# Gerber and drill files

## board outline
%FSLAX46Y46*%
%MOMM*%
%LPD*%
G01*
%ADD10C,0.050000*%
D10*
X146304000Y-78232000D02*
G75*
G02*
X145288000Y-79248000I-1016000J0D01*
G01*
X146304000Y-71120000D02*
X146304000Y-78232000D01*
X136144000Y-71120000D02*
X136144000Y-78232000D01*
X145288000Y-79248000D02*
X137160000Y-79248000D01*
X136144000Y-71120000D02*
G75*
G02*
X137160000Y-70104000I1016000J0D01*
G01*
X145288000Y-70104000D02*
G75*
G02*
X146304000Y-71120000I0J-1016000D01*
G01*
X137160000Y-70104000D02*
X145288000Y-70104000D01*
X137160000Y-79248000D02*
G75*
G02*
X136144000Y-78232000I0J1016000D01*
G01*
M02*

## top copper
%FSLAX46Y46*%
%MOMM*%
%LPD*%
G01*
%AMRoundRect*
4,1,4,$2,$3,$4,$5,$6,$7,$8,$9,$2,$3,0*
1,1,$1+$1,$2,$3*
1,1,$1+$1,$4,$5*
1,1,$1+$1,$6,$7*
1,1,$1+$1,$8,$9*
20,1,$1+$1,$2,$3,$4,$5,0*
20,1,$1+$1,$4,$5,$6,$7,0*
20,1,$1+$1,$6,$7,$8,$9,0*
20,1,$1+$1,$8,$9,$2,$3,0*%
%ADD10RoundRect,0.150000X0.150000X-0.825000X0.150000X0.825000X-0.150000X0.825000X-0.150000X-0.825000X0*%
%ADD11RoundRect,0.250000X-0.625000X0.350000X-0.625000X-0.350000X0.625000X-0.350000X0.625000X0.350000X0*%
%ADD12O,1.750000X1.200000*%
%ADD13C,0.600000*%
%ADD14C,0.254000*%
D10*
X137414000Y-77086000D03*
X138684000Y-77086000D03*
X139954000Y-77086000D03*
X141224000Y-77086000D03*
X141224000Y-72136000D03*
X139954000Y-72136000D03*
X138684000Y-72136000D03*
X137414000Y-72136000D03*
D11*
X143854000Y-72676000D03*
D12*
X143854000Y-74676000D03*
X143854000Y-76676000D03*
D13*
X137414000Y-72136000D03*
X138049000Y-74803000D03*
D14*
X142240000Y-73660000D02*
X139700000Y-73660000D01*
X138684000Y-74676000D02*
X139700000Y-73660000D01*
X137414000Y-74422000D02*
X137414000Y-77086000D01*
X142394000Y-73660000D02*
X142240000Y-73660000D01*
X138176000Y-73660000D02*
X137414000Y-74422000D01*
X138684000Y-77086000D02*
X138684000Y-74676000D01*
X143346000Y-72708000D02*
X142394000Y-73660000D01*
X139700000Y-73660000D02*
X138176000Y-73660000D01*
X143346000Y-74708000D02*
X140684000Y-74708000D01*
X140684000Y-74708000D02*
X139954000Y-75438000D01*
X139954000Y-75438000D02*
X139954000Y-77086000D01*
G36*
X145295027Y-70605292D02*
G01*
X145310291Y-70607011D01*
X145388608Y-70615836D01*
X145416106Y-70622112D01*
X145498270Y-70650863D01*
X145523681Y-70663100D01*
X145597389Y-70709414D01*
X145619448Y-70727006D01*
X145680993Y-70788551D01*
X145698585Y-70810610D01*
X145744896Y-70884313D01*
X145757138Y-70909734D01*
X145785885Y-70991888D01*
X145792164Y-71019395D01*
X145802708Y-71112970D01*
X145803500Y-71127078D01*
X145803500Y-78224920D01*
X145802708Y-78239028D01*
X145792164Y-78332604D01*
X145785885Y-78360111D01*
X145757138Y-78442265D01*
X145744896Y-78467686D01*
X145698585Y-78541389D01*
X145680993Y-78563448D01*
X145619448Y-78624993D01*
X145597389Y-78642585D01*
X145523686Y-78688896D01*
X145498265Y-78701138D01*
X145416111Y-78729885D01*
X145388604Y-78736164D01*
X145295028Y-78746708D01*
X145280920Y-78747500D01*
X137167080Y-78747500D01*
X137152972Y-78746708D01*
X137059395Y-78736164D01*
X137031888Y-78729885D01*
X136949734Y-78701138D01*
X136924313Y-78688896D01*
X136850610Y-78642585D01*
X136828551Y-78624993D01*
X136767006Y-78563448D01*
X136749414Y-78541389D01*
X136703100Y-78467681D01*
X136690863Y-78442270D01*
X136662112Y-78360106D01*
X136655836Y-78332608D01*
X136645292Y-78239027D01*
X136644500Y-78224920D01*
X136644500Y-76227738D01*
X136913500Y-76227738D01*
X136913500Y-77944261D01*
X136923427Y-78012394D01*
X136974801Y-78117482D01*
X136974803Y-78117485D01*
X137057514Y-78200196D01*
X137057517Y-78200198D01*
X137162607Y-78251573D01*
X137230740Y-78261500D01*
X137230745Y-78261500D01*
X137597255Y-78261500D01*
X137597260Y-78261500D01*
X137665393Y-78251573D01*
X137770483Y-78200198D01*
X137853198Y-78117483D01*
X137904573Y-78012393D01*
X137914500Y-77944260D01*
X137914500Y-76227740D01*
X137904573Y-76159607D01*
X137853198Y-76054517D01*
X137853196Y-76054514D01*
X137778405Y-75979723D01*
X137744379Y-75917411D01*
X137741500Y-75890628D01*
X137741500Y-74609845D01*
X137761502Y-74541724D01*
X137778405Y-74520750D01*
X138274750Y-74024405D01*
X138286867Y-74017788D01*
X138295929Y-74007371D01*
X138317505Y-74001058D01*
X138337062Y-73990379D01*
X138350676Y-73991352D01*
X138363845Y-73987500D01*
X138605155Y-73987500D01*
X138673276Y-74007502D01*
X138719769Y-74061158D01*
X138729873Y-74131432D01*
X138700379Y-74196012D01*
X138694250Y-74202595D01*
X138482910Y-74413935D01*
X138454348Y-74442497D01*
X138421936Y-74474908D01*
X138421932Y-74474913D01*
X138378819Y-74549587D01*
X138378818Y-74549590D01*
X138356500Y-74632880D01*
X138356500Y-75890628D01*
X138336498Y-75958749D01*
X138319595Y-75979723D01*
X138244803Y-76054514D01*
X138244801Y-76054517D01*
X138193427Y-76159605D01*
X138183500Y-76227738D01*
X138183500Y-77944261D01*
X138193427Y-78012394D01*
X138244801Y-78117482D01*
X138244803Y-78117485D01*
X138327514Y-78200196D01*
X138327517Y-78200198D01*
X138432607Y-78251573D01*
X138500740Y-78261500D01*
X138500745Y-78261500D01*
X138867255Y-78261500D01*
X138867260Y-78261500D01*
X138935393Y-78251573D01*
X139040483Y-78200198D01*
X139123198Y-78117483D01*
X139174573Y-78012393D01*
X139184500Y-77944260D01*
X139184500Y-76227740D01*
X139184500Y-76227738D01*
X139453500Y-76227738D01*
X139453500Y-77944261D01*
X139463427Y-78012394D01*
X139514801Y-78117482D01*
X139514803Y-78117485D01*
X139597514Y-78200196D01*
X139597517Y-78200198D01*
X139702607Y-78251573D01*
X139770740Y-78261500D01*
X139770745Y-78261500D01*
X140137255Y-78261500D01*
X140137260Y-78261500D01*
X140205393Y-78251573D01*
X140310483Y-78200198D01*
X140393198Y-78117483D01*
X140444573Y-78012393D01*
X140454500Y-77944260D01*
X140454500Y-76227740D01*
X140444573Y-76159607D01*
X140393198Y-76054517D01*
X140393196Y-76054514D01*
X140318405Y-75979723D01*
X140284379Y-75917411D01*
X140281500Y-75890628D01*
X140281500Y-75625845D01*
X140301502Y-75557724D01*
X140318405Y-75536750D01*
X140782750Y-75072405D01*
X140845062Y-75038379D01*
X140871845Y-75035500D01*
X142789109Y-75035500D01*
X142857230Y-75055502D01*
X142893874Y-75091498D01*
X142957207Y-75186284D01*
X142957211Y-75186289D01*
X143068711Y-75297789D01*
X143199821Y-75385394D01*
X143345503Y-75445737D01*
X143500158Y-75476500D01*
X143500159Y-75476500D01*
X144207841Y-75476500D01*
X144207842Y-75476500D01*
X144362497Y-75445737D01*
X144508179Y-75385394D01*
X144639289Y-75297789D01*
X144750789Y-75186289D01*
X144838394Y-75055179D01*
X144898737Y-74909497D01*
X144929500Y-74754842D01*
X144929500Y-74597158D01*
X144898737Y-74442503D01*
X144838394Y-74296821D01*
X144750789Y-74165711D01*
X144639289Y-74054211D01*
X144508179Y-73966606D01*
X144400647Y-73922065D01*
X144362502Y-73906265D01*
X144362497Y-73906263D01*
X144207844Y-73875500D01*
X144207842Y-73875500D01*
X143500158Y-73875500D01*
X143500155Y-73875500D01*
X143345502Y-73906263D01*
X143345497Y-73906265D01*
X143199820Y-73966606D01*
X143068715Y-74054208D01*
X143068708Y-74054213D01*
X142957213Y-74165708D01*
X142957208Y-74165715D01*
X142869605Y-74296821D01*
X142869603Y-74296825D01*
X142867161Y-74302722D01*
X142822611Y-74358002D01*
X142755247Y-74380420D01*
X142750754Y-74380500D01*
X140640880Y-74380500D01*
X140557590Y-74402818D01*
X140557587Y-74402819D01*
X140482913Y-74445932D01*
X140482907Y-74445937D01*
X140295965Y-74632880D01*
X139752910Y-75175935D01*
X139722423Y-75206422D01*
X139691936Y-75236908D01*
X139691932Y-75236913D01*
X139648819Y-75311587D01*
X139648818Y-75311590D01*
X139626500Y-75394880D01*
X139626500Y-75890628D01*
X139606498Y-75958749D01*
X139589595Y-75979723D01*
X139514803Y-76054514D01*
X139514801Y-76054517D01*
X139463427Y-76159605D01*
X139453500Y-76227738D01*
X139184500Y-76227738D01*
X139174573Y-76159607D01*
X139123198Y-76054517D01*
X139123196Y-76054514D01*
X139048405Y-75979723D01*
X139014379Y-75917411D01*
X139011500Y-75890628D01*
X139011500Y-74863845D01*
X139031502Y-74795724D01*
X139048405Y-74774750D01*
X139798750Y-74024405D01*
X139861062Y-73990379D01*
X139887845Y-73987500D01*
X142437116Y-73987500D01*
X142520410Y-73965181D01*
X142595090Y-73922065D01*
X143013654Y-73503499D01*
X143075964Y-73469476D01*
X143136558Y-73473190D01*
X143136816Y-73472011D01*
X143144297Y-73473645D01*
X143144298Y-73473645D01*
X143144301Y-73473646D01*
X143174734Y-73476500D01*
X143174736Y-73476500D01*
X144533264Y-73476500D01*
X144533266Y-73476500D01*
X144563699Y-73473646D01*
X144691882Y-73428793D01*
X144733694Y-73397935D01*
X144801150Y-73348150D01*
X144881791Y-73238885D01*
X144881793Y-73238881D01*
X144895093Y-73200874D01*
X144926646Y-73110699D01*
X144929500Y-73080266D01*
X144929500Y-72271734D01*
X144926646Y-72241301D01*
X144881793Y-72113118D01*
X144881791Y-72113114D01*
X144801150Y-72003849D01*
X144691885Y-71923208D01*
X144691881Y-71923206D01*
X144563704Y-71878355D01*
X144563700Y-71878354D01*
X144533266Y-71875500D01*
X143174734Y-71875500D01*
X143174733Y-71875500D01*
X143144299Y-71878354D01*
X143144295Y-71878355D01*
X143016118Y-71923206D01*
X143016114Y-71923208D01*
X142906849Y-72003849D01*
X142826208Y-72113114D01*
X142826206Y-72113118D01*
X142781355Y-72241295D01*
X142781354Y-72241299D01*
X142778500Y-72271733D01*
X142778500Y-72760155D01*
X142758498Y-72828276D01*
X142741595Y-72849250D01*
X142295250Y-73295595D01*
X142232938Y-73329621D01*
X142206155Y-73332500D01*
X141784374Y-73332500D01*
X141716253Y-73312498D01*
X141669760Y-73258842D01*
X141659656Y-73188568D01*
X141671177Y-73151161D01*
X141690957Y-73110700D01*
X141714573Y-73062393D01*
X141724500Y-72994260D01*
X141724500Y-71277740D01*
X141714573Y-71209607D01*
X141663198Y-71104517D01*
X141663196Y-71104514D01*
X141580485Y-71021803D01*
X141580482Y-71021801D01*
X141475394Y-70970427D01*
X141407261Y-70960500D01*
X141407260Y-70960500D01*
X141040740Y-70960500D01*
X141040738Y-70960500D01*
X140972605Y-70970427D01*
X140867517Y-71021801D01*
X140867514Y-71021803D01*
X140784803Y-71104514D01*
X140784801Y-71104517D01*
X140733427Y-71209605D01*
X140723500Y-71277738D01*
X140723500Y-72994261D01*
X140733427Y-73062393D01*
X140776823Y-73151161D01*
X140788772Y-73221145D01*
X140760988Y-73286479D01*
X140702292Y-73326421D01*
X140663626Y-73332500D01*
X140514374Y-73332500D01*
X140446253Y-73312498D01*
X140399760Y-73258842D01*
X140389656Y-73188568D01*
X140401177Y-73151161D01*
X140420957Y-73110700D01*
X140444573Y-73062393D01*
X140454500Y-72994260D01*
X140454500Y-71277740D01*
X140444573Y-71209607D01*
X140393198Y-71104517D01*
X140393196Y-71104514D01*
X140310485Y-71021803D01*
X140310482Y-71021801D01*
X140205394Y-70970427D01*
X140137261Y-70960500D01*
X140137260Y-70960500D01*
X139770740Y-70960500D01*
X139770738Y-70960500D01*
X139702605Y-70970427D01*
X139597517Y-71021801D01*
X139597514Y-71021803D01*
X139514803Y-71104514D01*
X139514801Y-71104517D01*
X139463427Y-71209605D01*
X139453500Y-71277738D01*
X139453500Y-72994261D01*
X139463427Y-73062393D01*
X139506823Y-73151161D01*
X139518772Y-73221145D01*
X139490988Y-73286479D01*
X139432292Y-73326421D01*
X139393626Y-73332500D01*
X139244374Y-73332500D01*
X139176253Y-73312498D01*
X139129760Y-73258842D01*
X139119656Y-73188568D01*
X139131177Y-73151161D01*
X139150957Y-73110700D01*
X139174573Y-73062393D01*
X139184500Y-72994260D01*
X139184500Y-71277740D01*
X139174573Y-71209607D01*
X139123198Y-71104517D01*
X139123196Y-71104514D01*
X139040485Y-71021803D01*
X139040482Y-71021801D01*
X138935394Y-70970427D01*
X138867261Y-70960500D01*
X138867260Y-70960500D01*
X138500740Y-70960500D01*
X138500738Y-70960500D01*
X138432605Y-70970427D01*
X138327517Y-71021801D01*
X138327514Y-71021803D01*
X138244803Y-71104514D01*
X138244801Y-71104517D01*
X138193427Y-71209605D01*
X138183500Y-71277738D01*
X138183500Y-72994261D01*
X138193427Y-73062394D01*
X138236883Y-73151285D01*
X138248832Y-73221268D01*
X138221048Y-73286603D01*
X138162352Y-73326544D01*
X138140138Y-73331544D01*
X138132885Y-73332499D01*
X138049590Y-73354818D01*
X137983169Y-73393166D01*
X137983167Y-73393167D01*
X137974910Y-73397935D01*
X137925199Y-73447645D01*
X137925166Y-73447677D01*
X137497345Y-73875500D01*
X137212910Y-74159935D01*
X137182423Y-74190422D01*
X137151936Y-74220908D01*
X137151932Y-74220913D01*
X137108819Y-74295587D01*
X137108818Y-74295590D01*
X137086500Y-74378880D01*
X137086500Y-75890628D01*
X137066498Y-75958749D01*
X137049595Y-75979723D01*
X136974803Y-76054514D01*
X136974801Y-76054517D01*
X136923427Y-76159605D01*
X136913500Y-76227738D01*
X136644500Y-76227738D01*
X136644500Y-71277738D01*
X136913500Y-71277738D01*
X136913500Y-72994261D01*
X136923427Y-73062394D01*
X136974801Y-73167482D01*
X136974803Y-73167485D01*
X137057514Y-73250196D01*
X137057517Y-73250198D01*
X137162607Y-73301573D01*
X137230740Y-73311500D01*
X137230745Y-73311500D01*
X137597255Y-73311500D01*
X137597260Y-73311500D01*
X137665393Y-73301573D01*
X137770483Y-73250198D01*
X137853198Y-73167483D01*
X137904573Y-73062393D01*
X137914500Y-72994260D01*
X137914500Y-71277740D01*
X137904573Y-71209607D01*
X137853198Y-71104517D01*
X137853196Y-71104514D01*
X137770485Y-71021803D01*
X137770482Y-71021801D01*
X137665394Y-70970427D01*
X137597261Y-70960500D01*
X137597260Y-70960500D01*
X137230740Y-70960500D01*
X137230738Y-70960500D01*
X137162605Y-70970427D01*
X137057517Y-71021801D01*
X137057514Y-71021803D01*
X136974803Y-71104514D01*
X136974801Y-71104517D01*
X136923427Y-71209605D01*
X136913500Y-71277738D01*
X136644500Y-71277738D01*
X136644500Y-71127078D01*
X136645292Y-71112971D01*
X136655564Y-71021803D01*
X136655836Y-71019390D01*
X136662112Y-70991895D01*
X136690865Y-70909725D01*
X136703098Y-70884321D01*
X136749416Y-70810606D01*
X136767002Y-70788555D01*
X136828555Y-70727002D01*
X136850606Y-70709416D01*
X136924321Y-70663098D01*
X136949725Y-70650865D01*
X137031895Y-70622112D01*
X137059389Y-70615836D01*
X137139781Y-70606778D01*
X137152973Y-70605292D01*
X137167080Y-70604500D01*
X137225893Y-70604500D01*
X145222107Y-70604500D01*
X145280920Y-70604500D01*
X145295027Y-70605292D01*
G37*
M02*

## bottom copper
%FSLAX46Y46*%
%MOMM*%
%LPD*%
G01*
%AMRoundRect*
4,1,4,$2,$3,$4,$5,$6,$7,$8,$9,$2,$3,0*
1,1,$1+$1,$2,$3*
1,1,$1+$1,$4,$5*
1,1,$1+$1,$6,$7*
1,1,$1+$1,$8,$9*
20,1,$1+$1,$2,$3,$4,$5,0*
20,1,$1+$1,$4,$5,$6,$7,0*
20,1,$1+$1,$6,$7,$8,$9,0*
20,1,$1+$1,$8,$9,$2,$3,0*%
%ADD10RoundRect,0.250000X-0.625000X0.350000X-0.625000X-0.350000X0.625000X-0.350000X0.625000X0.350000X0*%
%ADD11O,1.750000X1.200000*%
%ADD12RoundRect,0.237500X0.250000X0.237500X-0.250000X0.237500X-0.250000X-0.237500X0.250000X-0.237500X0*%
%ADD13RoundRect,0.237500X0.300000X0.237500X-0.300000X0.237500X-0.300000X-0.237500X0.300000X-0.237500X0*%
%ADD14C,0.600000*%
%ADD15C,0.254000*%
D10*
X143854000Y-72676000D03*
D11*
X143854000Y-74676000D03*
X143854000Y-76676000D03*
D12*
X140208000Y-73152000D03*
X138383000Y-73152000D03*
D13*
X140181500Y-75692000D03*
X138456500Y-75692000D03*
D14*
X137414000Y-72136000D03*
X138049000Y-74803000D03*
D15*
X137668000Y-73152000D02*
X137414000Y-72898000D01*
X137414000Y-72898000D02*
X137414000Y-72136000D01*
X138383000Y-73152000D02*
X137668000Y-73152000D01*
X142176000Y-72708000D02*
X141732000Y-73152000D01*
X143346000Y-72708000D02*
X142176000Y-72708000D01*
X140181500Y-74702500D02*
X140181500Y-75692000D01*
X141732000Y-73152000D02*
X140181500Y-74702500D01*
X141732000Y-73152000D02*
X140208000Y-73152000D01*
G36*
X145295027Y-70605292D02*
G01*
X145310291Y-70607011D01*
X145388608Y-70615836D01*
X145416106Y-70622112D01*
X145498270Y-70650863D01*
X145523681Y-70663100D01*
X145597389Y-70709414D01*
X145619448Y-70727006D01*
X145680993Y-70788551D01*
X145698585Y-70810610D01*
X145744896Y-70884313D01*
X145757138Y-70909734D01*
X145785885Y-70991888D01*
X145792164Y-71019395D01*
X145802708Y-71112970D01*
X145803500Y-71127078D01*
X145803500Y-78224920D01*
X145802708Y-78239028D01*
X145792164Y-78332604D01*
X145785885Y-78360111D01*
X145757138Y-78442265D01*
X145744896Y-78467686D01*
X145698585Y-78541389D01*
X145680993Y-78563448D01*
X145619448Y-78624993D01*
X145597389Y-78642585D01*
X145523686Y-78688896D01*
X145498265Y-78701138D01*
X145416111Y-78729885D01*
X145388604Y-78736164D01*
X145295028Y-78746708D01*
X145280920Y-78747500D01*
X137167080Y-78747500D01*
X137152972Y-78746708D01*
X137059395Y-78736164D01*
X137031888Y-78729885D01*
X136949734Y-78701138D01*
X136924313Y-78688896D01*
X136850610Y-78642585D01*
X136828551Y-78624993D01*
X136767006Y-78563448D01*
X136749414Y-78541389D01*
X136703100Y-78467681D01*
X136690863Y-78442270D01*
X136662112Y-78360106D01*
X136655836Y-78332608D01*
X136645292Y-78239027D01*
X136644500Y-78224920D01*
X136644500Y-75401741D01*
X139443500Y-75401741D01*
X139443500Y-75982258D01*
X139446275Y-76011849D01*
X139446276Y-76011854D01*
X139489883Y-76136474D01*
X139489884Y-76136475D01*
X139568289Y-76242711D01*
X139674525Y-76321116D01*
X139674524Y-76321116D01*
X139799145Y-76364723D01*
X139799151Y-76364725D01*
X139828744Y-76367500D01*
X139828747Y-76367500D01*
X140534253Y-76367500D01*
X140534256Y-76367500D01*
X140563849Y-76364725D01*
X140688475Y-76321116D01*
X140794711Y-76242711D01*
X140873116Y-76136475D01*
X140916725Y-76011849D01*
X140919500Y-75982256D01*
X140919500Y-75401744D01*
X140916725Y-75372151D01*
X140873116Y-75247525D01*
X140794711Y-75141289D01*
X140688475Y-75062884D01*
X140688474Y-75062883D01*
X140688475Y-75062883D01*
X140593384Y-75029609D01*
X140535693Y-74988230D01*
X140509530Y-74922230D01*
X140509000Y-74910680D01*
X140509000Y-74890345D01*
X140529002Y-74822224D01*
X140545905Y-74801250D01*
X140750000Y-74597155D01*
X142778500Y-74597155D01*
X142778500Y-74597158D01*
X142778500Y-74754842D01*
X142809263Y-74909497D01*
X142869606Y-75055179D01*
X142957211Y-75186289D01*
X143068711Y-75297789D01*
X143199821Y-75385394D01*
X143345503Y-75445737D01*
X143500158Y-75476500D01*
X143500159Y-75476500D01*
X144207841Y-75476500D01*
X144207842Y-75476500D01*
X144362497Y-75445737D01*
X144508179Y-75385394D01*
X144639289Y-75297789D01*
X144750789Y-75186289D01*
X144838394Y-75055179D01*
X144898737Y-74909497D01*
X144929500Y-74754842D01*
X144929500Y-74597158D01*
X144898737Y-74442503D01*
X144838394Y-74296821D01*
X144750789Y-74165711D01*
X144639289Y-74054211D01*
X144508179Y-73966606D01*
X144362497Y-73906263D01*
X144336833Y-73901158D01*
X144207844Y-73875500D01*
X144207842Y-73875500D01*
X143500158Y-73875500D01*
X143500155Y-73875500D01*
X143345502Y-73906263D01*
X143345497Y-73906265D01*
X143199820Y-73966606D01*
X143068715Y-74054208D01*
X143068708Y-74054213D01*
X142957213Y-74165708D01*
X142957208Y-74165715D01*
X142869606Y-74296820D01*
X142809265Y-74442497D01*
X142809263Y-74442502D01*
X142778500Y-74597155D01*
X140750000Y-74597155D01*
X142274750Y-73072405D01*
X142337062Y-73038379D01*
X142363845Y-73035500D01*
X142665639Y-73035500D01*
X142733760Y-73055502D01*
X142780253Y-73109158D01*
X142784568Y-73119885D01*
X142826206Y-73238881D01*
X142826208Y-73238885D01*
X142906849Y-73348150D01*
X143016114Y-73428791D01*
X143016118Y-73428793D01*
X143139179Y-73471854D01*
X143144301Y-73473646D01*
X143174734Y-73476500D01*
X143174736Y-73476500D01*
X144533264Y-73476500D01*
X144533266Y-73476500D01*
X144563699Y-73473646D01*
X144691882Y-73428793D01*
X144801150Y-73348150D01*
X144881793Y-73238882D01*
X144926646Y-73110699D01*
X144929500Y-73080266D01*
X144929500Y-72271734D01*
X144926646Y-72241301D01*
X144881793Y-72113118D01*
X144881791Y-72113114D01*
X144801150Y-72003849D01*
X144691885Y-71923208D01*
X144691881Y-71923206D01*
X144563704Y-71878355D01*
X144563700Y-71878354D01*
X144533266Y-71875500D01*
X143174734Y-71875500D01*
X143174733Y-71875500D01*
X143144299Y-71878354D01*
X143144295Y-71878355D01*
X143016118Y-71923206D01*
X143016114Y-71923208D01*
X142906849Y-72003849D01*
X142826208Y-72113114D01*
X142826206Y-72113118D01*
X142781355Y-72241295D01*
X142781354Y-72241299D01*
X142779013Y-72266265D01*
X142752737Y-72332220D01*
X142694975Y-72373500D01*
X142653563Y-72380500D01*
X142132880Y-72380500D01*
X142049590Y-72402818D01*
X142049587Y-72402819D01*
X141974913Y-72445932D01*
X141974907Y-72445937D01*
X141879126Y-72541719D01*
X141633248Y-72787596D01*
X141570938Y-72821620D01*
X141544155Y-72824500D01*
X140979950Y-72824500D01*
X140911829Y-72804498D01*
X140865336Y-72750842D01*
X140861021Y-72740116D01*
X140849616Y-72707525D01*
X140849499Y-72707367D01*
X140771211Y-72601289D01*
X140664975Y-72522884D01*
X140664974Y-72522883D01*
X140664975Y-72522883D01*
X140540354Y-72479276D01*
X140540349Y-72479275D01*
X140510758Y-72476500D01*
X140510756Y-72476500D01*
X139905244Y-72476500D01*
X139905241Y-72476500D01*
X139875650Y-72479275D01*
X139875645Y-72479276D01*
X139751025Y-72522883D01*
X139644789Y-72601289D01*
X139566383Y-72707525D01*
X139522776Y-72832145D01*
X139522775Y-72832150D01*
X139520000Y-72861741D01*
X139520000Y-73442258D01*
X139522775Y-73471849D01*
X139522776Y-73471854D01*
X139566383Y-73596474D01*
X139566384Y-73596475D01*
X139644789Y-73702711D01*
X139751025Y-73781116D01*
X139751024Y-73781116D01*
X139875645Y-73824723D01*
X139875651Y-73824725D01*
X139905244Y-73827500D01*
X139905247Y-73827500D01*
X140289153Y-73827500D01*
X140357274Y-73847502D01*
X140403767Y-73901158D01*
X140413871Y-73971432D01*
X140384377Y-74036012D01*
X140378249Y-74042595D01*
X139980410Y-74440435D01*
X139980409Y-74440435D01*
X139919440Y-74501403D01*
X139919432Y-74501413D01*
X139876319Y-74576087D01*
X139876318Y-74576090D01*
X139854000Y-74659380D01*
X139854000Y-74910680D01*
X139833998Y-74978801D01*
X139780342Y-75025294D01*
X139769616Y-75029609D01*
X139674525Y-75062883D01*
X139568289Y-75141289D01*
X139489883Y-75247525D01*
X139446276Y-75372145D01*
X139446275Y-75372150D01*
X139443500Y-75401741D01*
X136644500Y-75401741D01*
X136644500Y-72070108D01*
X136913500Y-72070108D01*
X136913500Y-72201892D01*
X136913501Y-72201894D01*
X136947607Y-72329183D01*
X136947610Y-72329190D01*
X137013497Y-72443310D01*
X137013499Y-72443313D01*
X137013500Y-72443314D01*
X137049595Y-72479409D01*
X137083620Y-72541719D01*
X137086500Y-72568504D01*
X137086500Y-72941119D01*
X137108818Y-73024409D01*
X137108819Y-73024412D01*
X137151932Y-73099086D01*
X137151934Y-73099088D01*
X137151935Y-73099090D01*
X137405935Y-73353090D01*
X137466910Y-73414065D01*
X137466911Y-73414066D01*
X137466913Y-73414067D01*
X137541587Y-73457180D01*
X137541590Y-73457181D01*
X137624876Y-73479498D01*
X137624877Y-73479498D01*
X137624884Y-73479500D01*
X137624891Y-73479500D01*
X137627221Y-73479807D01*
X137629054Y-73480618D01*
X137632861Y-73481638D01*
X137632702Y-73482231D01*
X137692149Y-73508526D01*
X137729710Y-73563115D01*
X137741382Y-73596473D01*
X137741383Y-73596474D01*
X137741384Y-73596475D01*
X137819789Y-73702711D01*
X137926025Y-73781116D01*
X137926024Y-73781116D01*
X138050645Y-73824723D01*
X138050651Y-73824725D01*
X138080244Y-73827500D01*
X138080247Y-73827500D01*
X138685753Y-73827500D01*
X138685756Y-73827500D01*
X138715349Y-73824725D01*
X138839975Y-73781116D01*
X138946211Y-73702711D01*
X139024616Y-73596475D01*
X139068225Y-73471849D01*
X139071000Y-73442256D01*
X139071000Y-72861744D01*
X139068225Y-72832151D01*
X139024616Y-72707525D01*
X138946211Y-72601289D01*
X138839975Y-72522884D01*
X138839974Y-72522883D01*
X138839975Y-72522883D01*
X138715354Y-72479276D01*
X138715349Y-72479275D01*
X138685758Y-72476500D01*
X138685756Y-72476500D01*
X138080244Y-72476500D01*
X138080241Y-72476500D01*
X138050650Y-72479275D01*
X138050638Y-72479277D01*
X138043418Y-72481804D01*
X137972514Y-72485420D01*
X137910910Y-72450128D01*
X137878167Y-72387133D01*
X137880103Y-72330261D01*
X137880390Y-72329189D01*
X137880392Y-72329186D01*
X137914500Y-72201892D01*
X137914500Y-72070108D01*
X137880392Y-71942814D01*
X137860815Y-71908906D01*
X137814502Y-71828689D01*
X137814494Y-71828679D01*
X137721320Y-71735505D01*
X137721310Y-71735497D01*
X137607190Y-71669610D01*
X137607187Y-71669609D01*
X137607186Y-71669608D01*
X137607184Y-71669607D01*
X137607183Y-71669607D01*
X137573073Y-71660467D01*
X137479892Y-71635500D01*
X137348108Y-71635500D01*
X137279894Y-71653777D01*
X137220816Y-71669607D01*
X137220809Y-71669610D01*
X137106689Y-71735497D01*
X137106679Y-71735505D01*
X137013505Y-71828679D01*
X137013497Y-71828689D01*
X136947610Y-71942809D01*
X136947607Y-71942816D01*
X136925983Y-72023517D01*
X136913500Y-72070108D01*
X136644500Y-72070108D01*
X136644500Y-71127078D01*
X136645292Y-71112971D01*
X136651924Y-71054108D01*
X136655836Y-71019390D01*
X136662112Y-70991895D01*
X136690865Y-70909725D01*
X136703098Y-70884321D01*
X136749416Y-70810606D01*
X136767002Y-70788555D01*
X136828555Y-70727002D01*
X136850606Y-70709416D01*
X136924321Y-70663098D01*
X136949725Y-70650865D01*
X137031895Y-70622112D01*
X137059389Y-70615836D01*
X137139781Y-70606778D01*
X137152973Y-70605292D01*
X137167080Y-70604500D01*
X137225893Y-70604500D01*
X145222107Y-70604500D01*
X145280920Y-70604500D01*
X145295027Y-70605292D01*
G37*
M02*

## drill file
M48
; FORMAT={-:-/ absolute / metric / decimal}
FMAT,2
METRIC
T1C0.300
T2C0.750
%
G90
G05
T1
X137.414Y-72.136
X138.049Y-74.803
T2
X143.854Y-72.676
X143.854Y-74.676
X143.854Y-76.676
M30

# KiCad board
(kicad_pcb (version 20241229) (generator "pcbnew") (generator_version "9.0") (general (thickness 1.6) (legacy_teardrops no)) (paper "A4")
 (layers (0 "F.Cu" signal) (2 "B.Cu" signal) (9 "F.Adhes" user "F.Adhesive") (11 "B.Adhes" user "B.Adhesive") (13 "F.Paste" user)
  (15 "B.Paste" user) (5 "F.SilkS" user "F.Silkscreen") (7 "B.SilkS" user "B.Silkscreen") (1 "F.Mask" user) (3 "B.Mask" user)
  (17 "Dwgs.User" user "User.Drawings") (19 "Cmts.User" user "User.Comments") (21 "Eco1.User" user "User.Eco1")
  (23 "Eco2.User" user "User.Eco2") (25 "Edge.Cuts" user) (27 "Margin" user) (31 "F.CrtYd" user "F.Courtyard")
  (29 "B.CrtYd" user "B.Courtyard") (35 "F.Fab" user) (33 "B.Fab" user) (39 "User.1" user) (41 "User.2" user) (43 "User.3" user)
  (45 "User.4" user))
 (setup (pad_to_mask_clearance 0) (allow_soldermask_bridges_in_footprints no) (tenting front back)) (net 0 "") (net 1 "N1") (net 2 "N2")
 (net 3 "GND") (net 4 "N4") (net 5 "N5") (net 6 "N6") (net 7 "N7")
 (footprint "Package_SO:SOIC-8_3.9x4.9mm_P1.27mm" (layer "F.Cu") (at 139.319 74.611 90)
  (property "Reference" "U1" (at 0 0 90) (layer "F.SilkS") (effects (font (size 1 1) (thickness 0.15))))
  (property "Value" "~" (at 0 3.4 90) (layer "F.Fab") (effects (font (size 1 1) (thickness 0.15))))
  (pad "1" smd roundrect (at -2.475 -1.905 90) (size 1.95 0.6) (layers "F.Cu" "F.Mask" "F.Paste") (roundrect_rratio 0.25) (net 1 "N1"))
  (pad "2" smd roundrect (at -2.475 -0.635 90) (size 1.95 0.6) (layers "F.Cu" "F.Mask" "F.Paste") (roundrect_rratio 0.25) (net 1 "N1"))
  (pad "3" smd roundrect (at -2.475 0.635 90) (size 1.95 0.6) (layers "F.Cu" "F.Mask" "F.Paste") (roundrect_rratio 0.25) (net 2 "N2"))
  (pad "4" smd roundrect (at -2.475 1.905 90) (size 1.95 0.6) (layers "F.Cu" "F.Mask" "F.Paste") (roundrect_rratio 0.25) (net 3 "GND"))
  (pad "5" smd roundrect (at 2.475 1.905 90) (size 1.95 0.6) (layers "F.Cu" "F.Mask" "F.Paste") (roundrect_rratio 0.25) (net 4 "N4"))
  (pad "6" smd roundrect (at 2.475 0.635 90) (size 1.95 0.6) (layers "F.Cu" "F.Mask" "F.Paste") (roundrect_rratio 0.25) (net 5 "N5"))
  (pad "7" smd roundrect (at 2.475 -0.635 90) (size 1.95 0.6) (layers "F.Cu" "F.Mask" "F.Paste") (roundrect_rratio 0.25) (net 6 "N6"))
  (pad "8" smd roundrect (at 2.475 -1.905 90) (size 1.95 0.6) (layers "F.Cu" "F.Mask" "F.Paste") (roundrect_rratio 0.25) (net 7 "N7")))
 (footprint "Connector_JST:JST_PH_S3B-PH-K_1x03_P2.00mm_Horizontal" (layer "B.Cu") (at 143.854 72.676 -90)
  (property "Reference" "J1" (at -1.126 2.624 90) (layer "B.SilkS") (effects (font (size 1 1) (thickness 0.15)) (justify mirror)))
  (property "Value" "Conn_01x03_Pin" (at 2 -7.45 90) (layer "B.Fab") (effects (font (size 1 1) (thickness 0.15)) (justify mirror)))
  (pad "1" thru_hole roundrect (at 0 0 270) (size 1.2 1.75) (drill 0.75) (layers "*.Cu" "*.Mask") (remove_unused_layers no)
   (roundrect_rratio 0.208333) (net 1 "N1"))
  (pad "2" thru_hole oval (at 2 0 270) (size 1.2 1.75) (drill 0.75) (layers "*.Cu" "*.Mask") (remove_unused_layers no) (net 2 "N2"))
  (pad "3" thru_hole oval (at 4 0 270) (size 1.2 1.75) (drill 0.75) (layers "*.Cu" "*.Mask") (remove_unused_layers no) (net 3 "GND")))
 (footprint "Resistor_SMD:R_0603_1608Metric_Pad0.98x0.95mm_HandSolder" (layer "B.Cu") (at 139.2955 73.152 180)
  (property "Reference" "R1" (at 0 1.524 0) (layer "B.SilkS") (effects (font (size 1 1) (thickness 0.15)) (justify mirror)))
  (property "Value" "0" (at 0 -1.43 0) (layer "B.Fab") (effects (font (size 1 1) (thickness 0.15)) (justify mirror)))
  (pad "1" smd roundrect (at -0.9125 0 180) (size 0.975 0.95) (layers "B.Cu" "B.Mask" "B.Paste") (roundrect_rratio 0.25) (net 1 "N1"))
  (pad "2" smd roundrect (at 0.9125 0 180) (size 0.975 0.95) (layers "B.Cu" "B.Mask" "B.Paste") (roundrect_rratio 0.25) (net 7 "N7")))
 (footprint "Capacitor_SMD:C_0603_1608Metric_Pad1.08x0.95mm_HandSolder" (layer "B.Cu") (at 139.319 75.692 180)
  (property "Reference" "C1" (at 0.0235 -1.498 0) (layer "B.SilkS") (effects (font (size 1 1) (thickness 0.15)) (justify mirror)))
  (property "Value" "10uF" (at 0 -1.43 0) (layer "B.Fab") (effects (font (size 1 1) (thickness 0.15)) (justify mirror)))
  (pad "1" smd roundrect (at -0.8625 0 180) (size 1.075 0.95) (layers "B.Cu" "B.Mask" "B.Paste") (roundrect_rratio 0.25) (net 1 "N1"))
  (pad "2" smd roundrect (at 0.8625 0 180) (size 1.075 0.95) (layers "B.Cu" "B.Mask" "B.Paste") (roundrect_rratio 0.25) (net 3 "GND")))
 (gr_arc (start 146.304 78.232) (mid 146.00642 78.95042) (end 145.288 79.248) (stroke (width 0.05) (type default)) (layer "Edge.Cuts"))
 (gr_line (start 146.304 71.12) (end 146.304 78.232) (stroke (width 0.05) (type default)) (layer "Edge.Cuts"))
 (gr_line (start 136.144 71.12) (end 136.144 78.232) (stroke (width 0.05) (type default)) (layer "Edge.Cuts"))
 (gr_line (start 145.288 79.248) (end 137.16 79.248) (stroke (width 0.05) (type default)) (layer "Edge.Cuts"))
 (gr_arc (start 136.144 71.12) (mid 136.44158 70.40158) (end 137.16 70.104) (stroke (width 0.05) (type default)) (layer "Edge.Cuts"))
 (gr_arc (start 145.288 70.104) (mid 146.00642 70.40158) (end 146.304 71.12) (stroke (width 0.05) (type default)) (layer "Edge.Cuts"))
 (gr_line (start 137.16 70.104) (end 145.288 70.104) (stroke (width 0.05) (type default)) (layer "Edge.Cuts"))
 (gr_arc (start 137.16 79.248) (mid 136.44158 78.95042) (end 136.144 78.232) (stroke (width 0.05) (type default)) (layer "Edge.Cuts"))
 (via (at 137.414 72.136) (size 0.6) (drill 0.3) (layers "F.Cu" "B.Cu") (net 7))
 (segment (start 137.668 73.152) (end 137.414 72.898) (width 0.254) (layer "B.Cu") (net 7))
 (segment (start 137.414 72.898) (end 137.414 72.136) (width 0.254) (layer "B.Cu") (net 7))
 (segment (start 138.383 73.152) (end 137.668 73.152) (width 0.254) (layer "B.Cu") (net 7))
 (via (at 138.049 74.803) (size 0.6) (drill 0.3) (layers "F.Cu" "B.Cu") (free yes) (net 3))
 (segment (start 142.24 73.66) (end 139.7 73.66) (width 0.254) (layer "F.Cu") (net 1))
 (segment (start 138.684 74.676) (end 139.7 73.66) (width 0.254) (layer "F.Cu") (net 1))
 (segment (start 137.414 74.422) (end 137.414 77.086) (width 0.254) (layer "F.Cu") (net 1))
 (segment (start 142.394 73.66) (end 142.24 73.66) (width 0.254) (layer "F.Cu") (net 1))
 (segment (start 138.176 73.66) (end 137.414 74.422) (width 0.254) (layer "F.Cu") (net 1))
 (segment (start 138.684 77.086) (end 138.684 74.676) (width 0.254) (layer "F.Cu") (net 1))
 (segment (start 143.346 72.708) (end 142.394 73.66) (width 0.254) (layer "F.Cu") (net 1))
 (segment (start 139.7 73.66) (end 138.176 73.66) (width 0.254) (layer "F.Cu") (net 1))
 (segment (start 142.176 72.708) (end 141.732 73.152) (width 0.254) (layer "B.Cu") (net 1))
 (segment (start 143.346 72.708) (end 142.176 72.708) (width 0.254) (layer "B.Cu") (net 1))
 (segment (start 140.1815 74.7025) (end 140.1815 75.692) (width 0.254) (layer "B.Cu") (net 1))
 (segment (start 141.732 73.152) (end 140.1815 74.7025) (width 0.254) (layer "B.Cu") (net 1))
 (segment (start 141.732 73.152) (end 140.208 73.152) (width 0.254) (layer "B.Cu") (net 1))
 (segment (start 143.346 74.708) (end 140.684 74.708) (width 0.254) (layer "F.Cu") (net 2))
 (segment (start 140.684 74.708) (end 139.954 75.438) (width 0.254) (layer "F.Cu") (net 2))
 (segment (start 139.954 75.438) (end 139.954 77.086) (width 0.254) (layer "F.Cu") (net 2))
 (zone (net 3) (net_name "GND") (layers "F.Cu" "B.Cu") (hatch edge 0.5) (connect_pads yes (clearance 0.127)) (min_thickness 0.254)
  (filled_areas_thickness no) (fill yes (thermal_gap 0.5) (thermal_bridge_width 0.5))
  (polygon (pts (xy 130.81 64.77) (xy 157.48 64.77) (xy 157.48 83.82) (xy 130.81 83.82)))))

